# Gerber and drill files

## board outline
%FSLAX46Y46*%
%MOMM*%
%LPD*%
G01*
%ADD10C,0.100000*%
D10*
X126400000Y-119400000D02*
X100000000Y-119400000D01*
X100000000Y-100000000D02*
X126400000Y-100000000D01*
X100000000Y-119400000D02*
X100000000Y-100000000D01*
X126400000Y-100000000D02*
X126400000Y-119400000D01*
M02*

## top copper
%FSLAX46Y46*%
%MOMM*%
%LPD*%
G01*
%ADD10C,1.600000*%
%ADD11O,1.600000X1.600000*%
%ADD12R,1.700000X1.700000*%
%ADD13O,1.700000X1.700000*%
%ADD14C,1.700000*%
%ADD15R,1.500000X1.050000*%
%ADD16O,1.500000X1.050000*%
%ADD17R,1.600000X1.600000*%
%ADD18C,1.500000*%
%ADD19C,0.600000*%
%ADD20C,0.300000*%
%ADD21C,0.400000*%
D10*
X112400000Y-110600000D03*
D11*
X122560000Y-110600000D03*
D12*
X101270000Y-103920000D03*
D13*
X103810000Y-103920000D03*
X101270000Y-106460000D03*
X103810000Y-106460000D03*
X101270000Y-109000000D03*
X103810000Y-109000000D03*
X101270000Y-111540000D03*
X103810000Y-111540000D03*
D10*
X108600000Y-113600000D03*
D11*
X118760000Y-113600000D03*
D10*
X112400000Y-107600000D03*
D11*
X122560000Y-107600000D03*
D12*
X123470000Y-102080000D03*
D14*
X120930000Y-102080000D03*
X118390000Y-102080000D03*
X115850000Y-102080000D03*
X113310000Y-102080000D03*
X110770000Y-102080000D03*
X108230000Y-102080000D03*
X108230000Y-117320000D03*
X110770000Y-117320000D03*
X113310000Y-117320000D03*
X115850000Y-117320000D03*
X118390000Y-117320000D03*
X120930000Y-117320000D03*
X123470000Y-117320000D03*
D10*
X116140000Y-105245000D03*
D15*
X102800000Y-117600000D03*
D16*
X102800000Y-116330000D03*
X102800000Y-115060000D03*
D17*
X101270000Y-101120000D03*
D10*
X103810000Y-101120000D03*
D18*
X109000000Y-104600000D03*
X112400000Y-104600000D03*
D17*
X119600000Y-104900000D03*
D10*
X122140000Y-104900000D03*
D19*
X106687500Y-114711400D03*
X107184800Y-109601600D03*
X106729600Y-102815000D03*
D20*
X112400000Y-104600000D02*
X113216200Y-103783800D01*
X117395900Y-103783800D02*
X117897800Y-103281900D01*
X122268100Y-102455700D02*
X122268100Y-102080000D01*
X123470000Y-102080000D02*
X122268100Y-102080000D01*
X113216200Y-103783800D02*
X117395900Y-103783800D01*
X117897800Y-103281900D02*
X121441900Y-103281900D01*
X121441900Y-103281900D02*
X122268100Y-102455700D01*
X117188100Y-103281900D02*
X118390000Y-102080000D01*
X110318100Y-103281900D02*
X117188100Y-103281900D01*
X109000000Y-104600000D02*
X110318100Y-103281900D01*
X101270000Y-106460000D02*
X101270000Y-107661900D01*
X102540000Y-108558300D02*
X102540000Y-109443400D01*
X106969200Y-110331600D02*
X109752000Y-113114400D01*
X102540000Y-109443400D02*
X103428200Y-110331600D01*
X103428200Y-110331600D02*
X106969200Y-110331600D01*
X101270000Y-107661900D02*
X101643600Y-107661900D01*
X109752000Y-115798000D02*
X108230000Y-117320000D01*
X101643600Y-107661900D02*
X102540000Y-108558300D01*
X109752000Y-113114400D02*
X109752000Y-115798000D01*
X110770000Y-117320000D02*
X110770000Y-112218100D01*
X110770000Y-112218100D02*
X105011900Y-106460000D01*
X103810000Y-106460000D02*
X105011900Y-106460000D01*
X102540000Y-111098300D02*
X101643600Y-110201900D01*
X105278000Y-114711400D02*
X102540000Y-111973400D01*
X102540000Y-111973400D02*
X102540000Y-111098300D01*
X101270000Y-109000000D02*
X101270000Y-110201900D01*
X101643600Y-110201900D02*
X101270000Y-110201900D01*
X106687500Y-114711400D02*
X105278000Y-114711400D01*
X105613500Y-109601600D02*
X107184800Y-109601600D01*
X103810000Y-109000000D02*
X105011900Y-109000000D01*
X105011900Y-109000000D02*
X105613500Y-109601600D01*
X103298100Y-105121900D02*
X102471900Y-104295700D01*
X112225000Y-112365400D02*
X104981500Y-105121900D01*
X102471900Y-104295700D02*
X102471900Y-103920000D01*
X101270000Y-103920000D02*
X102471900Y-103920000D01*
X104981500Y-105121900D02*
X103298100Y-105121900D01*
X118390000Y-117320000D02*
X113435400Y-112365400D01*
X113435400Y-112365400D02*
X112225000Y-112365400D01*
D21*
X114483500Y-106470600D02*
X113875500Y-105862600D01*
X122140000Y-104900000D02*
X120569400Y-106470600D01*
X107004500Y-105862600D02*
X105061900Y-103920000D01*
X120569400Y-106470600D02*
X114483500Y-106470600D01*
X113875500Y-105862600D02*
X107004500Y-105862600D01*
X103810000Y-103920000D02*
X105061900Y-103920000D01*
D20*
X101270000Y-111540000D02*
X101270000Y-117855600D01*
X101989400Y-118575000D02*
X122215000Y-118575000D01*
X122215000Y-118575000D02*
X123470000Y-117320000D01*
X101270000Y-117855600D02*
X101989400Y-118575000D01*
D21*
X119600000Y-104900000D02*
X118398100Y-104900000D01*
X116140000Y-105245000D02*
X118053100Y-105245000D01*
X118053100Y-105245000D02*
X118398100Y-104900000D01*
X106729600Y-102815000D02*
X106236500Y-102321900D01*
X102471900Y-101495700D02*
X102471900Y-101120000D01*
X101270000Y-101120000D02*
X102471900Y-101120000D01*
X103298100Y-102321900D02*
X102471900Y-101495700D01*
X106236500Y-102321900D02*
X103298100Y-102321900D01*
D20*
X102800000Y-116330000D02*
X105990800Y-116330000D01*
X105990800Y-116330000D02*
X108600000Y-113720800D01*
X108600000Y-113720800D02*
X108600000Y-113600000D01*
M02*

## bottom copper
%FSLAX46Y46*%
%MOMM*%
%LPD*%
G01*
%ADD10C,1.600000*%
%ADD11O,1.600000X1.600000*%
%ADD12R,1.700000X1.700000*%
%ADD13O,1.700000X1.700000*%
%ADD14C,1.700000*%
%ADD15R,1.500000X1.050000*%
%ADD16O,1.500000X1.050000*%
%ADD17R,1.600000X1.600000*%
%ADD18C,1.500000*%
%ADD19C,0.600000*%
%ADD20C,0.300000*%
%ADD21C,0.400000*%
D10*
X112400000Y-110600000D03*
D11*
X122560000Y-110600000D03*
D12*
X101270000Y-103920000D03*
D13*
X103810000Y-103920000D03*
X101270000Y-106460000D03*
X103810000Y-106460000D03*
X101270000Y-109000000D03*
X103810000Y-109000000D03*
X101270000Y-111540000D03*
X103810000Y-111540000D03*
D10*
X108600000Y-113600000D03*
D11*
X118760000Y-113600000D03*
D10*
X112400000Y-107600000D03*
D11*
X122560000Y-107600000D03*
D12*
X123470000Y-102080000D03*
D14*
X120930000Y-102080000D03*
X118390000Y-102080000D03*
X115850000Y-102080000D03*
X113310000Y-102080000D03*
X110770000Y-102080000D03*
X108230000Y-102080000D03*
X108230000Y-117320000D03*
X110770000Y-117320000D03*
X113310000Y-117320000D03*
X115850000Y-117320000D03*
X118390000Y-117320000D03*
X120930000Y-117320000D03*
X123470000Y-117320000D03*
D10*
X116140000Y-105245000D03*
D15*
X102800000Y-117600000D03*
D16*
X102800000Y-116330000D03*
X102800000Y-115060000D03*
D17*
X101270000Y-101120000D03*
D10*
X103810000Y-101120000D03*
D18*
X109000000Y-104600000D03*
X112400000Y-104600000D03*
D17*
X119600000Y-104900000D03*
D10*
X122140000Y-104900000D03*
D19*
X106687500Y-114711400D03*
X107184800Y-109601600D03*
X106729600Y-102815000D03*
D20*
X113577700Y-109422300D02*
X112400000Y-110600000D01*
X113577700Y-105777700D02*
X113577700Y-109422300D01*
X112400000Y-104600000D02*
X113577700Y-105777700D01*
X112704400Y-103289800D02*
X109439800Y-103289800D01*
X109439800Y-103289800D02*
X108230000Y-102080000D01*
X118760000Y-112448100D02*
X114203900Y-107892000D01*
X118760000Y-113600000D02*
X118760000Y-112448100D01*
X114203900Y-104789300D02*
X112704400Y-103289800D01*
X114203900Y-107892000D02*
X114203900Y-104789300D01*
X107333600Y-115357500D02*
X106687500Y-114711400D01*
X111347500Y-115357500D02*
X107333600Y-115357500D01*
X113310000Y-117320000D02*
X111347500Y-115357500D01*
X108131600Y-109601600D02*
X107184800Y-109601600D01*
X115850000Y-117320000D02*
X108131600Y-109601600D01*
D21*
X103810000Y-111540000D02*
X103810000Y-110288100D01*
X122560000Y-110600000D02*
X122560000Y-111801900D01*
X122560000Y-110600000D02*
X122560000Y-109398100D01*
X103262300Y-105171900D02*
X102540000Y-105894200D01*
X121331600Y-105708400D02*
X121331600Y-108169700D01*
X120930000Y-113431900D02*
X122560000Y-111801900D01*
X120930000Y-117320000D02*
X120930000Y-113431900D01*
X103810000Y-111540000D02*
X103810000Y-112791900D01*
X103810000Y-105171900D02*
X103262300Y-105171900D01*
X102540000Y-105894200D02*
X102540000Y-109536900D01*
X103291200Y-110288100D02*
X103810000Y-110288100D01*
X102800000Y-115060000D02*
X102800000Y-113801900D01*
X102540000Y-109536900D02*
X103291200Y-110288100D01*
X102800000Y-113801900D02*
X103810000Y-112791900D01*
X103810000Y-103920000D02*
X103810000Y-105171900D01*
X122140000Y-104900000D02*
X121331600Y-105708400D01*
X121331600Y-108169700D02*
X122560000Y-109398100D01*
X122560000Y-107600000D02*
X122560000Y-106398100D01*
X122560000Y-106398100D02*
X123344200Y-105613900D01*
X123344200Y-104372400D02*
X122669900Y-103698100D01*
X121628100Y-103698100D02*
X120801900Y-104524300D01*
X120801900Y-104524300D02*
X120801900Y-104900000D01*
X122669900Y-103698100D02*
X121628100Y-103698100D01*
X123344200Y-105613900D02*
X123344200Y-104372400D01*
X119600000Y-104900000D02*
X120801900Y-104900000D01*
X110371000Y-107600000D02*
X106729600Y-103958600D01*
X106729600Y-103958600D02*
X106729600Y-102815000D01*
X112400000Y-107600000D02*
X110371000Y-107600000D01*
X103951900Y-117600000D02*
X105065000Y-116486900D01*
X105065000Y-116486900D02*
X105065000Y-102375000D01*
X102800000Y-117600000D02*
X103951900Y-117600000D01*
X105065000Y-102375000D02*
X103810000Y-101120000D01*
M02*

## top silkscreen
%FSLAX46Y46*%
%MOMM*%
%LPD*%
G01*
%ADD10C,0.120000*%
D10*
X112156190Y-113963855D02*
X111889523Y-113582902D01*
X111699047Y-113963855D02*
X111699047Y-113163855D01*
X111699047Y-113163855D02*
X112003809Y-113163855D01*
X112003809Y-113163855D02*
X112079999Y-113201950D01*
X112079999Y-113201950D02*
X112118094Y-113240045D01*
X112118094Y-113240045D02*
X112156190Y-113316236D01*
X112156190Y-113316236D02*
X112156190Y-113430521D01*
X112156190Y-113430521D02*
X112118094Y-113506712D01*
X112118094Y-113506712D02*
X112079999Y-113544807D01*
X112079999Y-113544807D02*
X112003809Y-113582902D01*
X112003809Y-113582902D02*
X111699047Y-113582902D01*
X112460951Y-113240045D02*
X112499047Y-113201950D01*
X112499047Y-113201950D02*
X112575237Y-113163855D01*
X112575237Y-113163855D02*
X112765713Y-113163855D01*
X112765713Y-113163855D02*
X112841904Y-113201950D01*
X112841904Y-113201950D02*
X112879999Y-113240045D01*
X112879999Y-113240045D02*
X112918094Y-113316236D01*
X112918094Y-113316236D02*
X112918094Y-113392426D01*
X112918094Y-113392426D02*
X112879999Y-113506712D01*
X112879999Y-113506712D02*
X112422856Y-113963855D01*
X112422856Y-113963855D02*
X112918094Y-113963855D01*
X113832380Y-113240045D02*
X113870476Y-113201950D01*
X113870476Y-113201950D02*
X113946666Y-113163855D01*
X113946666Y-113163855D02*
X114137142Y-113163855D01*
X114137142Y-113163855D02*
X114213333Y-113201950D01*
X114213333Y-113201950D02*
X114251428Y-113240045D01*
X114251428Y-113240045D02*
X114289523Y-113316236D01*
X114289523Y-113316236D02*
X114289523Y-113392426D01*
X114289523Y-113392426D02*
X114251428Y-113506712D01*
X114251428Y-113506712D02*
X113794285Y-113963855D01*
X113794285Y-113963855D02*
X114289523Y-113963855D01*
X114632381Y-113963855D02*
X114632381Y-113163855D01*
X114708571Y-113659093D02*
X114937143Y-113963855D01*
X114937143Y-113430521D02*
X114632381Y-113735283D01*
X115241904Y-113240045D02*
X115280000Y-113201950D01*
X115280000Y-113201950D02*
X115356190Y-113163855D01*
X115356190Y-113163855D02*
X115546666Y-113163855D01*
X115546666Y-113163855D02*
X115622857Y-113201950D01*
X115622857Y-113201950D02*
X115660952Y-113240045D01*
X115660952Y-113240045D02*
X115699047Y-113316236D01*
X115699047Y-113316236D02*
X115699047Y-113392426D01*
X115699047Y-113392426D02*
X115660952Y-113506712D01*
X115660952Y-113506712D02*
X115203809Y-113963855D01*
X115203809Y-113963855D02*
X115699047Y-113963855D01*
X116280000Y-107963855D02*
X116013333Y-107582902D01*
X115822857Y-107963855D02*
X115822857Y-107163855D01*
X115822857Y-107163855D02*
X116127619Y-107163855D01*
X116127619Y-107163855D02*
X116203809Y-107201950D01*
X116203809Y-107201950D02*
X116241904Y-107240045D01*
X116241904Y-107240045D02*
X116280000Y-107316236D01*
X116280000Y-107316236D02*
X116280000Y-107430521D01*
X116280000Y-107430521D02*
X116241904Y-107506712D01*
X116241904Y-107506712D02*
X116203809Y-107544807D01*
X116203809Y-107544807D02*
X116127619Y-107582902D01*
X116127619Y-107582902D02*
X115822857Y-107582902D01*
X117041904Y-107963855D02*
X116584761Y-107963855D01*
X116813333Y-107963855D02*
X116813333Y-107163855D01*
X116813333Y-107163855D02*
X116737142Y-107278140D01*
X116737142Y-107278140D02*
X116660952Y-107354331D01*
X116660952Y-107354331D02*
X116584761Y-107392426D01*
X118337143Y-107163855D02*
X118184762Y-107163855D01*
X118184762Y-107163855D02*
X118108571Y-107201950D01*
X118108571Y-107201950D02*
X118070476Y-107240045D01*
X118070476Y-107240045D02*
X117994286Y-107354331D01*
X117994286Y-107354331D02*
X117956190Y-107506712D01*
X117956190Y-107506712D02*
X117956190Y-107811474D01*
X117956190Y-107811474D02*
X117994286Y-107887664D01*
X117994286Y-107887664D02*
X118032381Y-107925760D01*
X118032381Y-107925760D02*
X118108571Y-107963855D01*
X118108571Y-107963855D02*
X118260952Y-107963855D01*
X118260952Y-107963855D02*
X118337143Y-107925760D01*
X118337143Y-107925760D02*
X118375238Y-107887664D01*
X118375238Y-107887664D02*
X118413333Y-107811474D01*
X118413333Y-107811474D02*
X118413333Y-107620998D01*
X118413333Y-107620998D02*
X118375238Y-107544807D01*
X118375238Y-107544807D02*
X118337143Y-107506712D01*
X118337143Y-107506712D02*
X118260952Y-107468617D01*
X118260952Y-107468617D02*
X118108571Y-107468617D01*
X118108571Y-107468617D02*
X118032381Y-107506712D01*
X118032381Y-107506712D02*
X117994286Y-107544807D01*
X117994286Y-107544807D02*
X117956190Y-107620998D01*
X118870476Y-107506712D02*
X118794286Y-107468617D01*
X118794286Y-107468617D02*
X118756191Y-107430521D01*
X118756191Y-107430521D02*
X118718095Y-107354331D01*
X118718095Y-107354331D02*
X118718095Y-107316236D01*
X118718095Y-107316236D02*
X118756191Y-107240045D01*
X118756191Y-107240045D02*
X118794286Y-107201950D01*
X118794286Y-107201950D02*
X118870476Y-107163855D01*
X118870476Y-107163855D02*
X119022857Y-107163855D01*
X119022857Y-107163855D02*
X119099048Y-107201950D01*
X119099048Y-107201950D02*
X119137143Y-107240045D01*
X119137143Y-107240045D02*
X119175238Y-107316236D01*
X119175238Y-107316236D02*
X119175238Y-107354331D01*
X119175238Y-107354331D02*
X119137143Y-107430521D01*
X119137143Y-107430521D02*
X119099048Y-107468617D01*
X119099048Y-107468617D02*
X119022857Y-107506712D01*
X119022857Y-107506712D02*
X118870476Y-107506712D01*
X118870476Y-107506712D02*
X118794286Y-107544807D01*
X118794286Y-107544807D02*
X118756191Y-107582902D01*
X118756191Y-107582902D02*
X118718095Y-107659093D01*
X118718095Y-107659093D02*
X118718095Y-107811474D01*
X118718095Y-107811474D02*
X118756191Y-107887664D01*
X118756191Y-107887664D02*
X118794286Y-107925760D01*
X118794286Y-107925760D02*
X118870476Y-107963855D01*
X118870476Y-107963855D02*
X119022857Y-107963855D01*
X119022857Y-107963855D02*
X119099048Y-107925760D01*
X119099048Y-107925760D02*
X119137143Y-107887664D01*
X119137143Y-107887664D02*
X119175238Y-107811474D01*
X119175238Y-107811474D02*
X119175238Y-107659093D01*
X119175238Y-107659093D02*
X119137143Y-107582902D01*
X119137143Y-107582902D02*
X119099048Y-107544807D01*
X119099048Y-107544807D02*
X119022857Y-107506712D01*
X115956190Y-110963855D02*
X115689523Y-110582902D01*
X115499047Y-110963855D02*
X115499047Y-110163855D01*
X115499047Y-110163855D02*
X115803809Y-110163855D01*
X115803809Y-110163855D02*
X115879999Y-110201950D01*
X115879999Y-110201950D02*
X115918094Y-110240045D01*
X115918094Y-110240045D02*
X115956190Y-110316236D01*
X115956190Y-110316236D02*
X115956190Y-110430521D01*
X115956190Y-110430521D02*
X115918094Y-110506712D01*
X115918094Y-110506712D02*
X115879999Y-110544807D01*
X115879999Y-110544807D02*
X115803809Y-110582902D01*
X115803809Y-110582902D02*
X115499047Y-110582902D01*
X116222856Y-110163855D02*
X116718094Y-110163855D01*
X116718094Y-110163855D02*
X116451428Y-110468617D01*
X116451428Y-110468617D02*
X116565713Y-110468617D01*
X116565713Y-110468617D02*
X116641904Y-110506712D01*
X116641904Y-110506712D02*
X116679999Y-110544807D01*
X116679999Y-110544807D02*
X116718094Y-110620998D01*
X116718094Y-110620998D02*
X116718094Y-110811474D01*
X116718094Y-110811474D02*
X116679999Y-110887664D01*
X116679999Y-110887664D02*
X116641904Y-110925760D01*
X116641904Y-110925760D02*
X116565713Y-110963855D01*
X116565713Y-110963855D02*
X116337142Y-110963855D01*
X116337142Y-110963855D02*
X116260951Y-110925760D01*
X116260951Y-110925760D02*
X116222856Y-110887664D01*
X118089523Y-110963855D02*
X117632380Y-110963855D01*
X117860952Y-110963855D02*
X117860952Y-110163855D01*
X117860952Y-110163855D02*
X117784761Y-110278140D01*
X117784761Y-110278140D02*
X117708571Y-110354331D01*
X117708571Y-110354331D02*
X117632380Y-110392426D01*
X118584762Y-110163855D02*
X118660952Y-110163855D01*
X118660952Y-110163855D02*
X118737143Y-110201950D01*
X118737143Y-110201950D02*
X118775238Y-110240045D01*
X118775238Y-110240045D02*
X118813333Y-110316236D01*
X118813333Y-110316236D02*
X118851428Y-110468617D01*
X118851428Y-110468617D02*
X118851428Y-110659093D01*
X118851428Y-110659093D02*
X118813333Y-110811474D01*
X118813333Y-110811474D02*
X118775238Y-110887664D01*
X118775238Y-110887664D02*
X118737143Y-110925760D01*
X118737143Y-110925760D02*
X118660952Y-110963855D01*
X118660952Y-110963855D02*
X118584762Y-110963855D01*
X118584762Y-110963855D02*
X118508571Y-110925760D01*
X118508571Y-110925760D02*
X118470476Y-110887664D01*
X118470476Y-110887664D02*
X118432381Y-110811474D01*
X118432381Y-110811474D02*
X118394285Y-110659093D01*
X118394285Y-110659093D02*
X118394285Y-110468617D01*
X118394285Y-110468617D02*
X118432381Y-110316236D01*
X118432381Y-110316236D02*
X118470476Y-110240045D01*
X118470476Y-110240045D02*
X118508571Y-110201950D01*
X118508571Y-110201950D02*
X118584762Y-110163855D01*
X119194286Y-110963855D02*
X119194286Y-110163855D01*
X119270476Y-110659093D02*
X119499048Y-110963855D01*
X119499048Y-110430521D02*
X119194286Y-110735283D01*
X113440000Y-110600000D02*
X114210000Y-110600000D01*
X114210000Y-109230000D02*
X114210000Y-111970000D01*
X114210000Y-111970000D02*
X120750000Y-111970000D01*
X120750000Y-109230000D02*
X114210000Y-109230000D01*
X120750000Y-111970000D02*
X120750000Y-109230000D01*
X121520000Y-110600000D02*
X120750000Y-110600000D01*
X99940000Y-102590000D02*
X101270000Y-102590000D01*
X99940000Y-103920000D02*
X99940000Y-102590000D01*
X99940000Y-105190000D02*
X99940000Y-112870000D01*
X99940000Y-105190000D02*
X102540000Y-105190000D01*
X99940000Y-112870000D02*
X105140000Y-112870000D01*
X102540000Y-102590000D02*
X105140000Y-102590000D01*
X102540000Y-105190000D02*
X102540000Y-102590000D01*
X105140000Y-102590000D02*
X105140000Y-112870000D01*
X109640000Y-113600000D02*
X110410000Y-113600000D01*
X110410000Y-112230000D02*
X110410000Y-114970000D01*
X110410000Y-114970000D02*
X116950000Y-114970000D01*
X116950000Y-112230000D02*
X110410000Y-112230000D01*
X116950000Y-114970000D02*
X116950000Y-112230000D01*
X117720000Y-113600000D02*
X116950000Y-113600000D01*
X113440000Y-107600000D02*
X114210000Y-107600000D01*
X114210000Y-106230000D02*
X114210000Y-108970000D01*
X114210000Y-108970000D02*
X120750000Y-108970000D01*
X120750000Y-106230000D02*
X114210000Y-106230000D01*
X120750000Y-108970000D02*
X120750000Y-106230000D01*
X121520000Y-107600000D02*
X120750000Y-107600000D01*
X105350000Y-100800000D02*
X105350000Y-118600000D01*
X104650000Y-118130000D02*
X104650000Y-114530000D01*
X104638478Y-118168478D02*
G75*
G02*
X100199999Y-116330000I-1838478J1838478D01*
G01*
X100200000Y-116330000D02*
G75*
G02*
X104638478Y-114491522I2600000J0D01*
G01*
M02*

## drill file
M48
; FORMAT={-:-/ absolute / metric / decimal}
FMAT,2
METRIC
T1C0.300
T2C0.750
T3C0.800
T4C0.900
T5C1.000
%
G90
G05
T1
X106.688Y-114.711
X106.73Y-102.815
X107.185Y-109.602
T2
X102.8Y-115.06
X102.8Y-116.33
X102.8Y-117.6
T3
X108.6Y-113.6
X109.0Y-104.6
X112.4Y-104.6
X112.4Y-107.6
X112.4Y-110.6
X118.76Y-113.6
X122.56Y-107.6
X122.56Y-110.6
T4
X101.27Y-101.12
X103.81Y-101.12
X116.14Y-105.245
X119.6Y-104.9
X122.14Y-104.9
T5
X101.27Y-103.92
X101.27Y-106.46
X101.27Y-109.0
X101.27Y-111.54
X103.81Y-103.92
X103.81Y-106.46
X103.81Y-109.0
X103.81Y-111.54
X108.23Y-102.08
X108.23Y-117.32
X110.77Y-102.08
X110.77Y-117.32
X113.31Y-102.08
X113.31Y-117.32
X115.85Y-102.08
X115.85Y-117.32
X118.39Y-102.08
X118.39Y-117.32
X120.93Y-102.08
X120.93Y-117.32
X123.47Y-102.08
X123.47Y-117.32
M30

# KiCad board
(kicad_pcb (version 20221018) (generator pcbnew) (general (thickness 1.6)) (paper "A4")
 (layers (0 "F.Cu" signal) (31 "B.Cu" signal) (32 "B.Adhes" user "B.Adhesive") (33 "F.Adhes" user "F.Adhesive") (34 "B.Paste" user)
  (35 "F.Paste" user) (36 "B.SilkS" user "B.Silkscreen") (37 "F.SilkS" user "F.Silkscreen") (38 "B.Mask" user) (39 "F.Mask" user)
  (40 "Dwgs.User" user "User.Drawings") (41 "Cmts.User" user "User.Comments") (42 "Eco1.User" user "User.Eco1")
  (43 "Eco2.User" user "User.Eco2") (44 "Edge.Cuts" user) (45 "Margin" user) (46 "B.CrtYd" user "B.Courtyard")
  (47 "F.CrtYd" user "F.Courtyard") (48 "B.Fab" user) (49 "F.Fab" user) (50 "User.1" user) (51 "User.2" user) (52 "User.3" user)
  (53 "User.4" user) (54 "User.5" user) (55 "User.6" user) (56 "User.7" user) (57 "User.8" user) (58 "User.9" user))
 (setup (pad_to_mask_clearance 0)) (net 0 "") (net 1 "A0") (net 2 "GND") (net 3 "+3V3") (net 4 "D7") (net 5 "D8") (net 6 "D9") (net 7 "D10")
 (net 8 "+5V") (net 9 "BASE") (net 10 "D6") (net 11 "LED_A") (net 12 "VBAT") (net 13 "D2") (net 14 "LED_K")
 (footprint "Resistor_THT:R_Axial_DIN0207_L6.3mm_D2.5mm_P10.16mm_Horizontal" (layer "F.Cu") (at 112.4 110.6)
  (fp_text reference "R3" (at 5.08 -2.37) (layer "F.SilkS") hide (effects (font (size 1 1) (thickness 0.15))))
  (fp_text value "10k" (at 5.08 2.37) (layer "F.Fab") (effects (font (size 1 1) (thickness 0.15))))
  (fp_line (start 1.04 0) (end 1.81 0) (stroke (width 0.12) (type solid)) (layer "F.SilkS"))
  (fp_line (start 1.81 -1.37) (end 1.81 1.37) (stroke (width 0.12) (type solid)) (layer "F.SilkS"))
  (fp_line (start 1.81 1.37) (end 8.35 1.37) (stroke (width 0.12) (type solid)) (layer "F.SilkS"))
  (fp_line (start 8.35 -1.37) (end 1.81 -1.37) (stroke (width 0.12) (type solid)) (layer "F.SilkS"))
  (fp_line (start 8.35 1.37) (end 8.35 -1.37) (stroke (width 0.12) (type solid)) (layer "F.SilkS"))
  (fp_line (start 9.12 0) (end 8.35 0) (stroke (width 0.12) (type solid)) (layer "F.SilkS"))
  (pad "1" thru_hole circle (at 0 0) (size 1.6 1.6) (drill 0.8) (layers "*.Cu" "*.Mask") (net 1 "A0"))
  (pad "2" thru_hole oval (at 10.16 0) (size 1.6 1.6) (drill 0.8) (layers "*.Cu" "*.Mask") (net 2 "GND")))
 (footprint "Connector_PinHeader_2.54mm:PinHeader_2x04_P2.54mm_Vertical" (layer "F.Cu") (at 101.27 103.92)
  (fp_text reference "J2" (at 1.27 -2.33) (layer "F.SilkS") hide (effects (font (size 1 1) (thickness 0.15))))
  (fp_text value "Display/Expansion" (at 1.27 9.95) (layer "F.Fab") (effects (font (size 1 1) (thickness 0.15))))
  (fp_line (start -1.33 -1.33) (end 0 -1.33) (stroke (width 0.12) (type solid)) (layer "F.SilkS"))
  (fp_line (start -1.33 0) (end -1.33 -1.33) (stroke (width 0.12) (type solid)) (layer "F.SilkS"))
  (fp_line (start -1.33 1.27) (end -1.33 8.95) (stroke (width 0.12) (type solid)) (layer "F.SilkS"))
  (fp_line (start -1.33 1.27) (end 1.27 1.27) (stroke (width 0.12) (type solid)) (layer "F.SilkS"))
  (fp_line (start -1.33 8.95) (end 3.87 8.95) (stroke (width 0.12) (type solid)) (layer "F.SilkS"))
  (fp_line (start 1.27 -1.33) (end 3.87 -1.33) (stroke (width 0.12) (type solid)) (layer "F.SilkS"))
  (fp_line (start 1.27 1.27) (end 1.27 -1.33) (stroke (width 0.12) (type solid)) (layer "F.SilkS"))
  (fp_line (start 3.87 -1.33) (end 3.87 8.95) (stroke (width 0.12) (type solid)) (layer "F.SilkS"))
  (pad "1" thru_hole rect (at 0 0) (size 1.7 1.7) (drill 1) (layers "*.Cu" "*.Mask") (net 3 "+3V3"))
  (pad "2" thru_hole oval (at 2.54 0) (size 1.7 1.7) (drill 1) (layers "*.Cu" "*.Mask") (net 2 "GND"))
  (pad "3" thru_hole oval (at 0 2.54) (size 1.7 1.7) (drill 1) (layers "*.Cu" "*.Mask") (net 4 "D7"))
  (pad "4" thru_hole oval (at 2.54 2.54) (size 1.7 1.7) (drill 1) (layers "*.Cu" "*.Mask") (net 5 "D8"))
  (pad "5" thru_hole oval (at 0 5.08) (size 1.7 1.7) (drill 1) (layers "*.Cu" "*.Mask") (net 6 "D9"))
  (pad "6" thru_hole oval (at 2.54 5.08) (size 1.7 1.7) (drill 1) (layers "*.Cu" "*.Mask") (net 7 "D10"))
  (pad "7" thru_hole oval (at 0 7.62) (size 1.7 1.7) (drill 1) (layers "*.Cu" "*.Mask") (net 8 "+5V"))
  (pad "8" thru_hole oval (at 2.54 7.62) (size 1.7 1.7) (drill 1) (layers "*.Cu" "*.Mask") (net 2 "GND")))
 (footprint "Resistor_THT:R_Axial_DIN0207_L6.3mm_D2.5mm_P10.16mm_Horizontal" (layer "F.Cu") (at 108.6 113.6)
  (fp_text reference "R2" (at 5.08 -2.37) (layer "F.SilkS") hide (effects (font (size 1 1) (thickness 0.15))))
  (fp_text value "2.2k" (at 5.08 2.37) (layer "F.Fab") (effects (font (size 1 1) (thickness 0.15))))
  (fp_line (start 1.04 0) (end 1.81 0) (stroke (width 0.12) (type solid)) (layer "F.SilkS"))
  (fp_line (start 1.81 -1.37) (end 1.81 1.37) (stroke (width 0.12) (type solid)) (layer "F.SilkS"))
  (fp_line (start 1.81 1.37) (end 8.35 1.37) (stroke (width 0.12) (type solid)) (layer "F.SilkS"))
  (fp_line (start 8.35 -1.37) (end 1.81 -1.37) (stroke (width 0.12) (type solid)) (layer "F.SilkS"))
  (fp_line (start 8.35 1.37) (end 8.35 -1.37) (stroke (width 0.12) (type solid)) (layer "F.SilkS"))
  (fp_line (start 9.12 0) (end 8.35 0) (stroke (width 0.12) (type solid)) (layer "F.SilkS"))
  (pad "1" thru_hole circle (at 0 0) (size 1.6 1.6) (drill 0.8) (layers "*.Cu" "*.Mask") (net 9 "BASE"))
  (pad "2" thru_hole oval (at 10.16 0) (size 1.6 1.6) (drill 0.8) (layers "*.Cu" "*.Mask") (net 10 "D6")))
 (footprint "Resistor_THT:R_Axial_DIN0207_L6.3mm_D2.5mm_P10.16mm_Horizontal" (layer "F.Cu") (at 112.4 107.6)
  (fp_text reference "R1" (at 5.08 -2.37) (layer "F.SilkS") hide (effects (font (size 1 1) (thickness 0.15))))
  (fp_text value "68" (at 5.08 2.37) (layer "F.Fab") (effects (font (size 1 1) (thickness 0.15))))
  (fp_line (start 1.04 0) (end 1.81 0) (stroke (width 0.12) (type solid)) (layer "F.SilkS"))
  (fp_line (start 1.81 -1.37) (end 1.81 1.37) (stroke (width 0.12) (type solid)) (layer "F.SilkS"))
  (fp_line (start 1.81 1.37) (end 8.35 1.37) (stroke (width 0.12) (type solid)) (layer "F.SilkS"))
  (fp_line (start 8.35 -1.37) (end 1.81 -1.37) (stroke (width 0.12) (type solid)) (layer "F.SilkS"))
  (fp_line (start 8.35 1.37) (end 8.35 -1.37) (stroke (width 0.12) (type solid)) (layer "F.SilkS"))
  (fp_line (start 9.12 0) (end 8.35 0) (stroke (width 0.12) (type solid)) (layer "F.SilkS"))
  (pad "1" thru_hole circle (at 0 0) (size 1.6 1.6) (drill 0.8) (layers "*.Cu" "*.Mask") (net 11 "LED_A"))
  (pad "2" thru_hole oval (at 10.16 0) (size 1.6 1.6) (drill 0.8) (layers "*.Cu" "*.Mask") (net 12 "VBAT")))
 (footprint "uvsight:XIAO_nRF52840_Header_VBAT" (layer "F.Cu") (at 115.85 109.7)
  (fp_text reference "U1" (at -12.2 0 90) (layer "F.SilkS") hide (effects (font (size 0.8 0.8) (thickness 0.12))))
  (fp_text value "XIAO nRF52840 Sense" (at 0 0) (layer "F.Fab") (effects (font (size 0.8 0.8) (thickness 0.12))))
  (fp_line (start -10.5 -8.9) (end -10.5 8.9) (stroke (width 0.12) (type solid)) (layer "F.SilkS"))
  (pad "1" thru_hole rect (at 7.62 -7.62) (size 1.7 1.7) (drill 1) (layers "*.Cu" "*.Mask") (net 1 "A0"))
  (pad "2" thru_hole circle (at 5.08 -7.62) (size 1.7 1.7) (drill 1) (layers "*.Cu" "*.Mask"))
  (pad "3" thru_hole circle (at 2.54 -7.62) (size 1.7 1.7) (drill 1) (layers "*.Cu" "*.Mask") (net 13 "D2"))
  (pad "4" thru_hole circle (at 0 -7.62) (size 1.7 1.7) (drill 1) (layers "*.Cu" "*.Mask"))
  (pad "5" thru_hole circle (at -2.54 -7.62) (size 1.7 1.7) (drill 1) (layers "*.Cu" "*.Mask"))
  (pad "6" thru_hole circle (at -5.08 -7.62) (size 1.7 1.7) (drill 1) (layers "*.Cu" "*.Mask"))
  (pad "7" thru_hole circle (at -7.62 -7.62) (size 1.7 1.7) (drill 1) (layers "*.Cu" "*.Mask") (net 10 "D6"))
  (pad "8" thru_hole circle (at -7.62 7.62) (size 1.7 1.7) (drill 1) (layers "*.Cu" "*.Mask") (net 4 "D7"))
  (pad "9" thru_hole circle (at -5.08 7.62) (size 1.7 1.7) (drill 1) (layers "*.Cu" "*.Mask") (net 5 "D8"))
  (pad "10" thru_hole circle (at -2.54 7.62) (size 1.7 1.7) (drill 1) (layers "*.Cu" "*.Mask") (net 6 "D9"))
  (pad "11" thru_hole circle (at 0 7.62) (size 1.7 1.7) (drill 1) (layers "*.Cu" "*.Mask") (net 7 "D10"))
  (pad "12" thru_hole circle (at 2.54 7.62) (size 1.7 1.7) (drill 1) (layers "*.Cu" "*.Mask") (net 3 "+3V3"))
  (pad "13" thru_hole circle (at 5.08 7.62) (size 1.7 1.7) (drill 1) (layers "*.Cu" "*.Mask") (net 2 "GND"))
  (pad "14" thru_hole circle (at 7.62 7.62) (size 1.7 1.7) (drill 1) (layers "*.Cu" "*.Mask") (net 8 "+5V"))
  (pad "15" thru_hole circle (at 0.29 -4.455) (size 1.6 1.6) (drill 0.9) (layers "*.Cu" "*.Mask") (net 12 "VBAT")))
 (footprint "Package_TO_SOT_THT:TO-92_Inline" (layer "F.Cu") (at 102.8 117.6 90)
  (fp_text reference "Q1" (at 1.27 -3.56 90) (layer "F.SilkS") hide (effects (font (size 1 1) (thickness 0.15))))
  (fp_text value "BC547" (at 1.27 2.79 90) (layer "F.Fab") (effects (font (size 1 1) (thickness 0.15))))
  (fp_line (start -0.53 1.85) (end 3.07 1.85) (stroke (width 0.12) (type solid)) (layer "F.SilkS"))
  (fp_arc (start -0.568478 1.838478) (mid -1.132087 -0.994977) (end 1.27 -2.6) (stroke (width 0.12) (type solid)) (layer "F.SilkS"))
  (fp_arc (start 1.27 -2.6) (mid 3.672087 -0.994977) (end 3.108478 1.838478) (stroke (width 0.12) (type solid)) (layer "F.SilkS"))
  (pad "1" thru_hole rect (at 0 0 90) (size 1.05 1.5) (drill 0.75) (layers "*.Cu" "*.Mask") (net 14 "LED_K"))
  (pad "2" thru_hole oval (at 1.27 0 90) (size 1.05 1.5) (drill 0.75) (layers "*.Cu" "*.Mask") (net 9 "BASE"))
  (pad "3" thru_hole oval (at 2.54 0 90) (size 1.05 1.5) (drill 0.75) (layers "*.Cu" "*.Mask") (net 2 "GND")))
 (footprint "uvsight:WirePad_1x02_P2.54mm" (layer "F.Cu") (at 101.27 101.12)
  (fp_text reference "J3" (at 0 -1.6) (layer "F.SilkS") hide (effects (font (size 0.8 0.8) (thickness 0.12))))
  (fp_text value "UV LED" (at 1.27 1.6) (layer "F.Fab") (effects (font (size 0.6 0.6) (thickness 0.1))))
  (pad "1" thru_hole rect (at 0 0) (size 1.6 1.6) (drill 0.9) (layers "*.Cu" "*.Mask") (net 11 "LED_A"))
  (pad "2" thru_hole circle (at 2.54 0) (size 1.6 1.6) (drill 0.9) (layers "*.Cu" "*.Mask") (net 14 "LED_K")))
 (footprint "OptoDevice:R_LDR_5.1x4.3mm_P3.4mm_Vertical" (layer "B.Cu") (at 109 104.6)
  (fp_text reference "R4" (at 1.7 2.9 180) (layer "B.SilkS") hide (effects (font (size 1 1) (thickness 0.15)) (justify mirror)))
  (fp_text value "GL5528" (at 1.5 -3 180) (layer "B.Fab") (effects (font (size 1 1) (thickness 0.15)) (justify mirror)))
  (pad "1" thru_hole circle (at 0 0) (size 1.5 1.5) (drill 0.8) (layers "*.Cu" "*.Mask") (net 13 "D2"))
  (pad "2" thru_hole circle (at 3.4 0) (size 1.5 1.5) (drill 0.8) (layers "*.Cu" "*.Mask") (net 1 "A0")))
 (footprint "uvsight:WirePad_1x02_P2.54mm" (layer "B.Cu") (at 119.6 104.9)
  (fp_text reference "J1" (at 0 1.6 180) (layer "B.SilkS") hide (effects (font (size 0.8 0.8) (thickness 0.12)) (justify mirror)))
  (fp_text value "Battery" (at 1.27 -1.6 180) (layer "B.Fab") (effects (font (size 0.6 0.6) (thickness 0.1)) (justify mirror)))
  (pad "1" thru_hole rect (at 0 0) (size 1.6 1.6) (drill 0.9) (layers "*.Cu" "*.Mask") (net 12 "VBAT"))
  (pad "2" thru_hole circle (at 2.54 0) (size 1.6 1.6) (drill 0.9) (layers "*.Cu" "*.Mask") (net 2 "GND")))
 (gr_line (start 126.4 119.4) (end 100 119.4) (stroke (width 0.1) (type default)) (layer "Edge.Cuts"))
 (gr_line (start 100 100) (end 126.4 100) (stroke (width 0.1) (type default)) (layer "Edge.Cuts"))
 (gr_line (start 100 119.4) (end 100 100) (stroke (width 0.1) (type default)) (layer "Edge.Cuts"))
 (gr_line (start 126.4 100) (end 126.4 119.4) (stroke (width 0.1) (type default)) (layer "Edge.Cuts"))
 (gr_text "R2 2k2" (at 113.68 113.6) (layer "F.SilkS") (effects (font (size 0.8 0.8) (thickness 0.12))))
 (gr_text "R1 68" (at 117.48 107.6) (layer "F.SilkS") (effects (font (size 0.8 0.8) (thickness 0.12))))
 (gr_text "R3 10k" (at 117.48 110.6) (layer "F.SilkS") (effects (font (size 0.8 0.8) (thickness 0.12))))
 (segment (start 112.4 104.6) (end 113.2162 103.7838) (width 0.3) (layer "F.Cu") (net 1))
 (segment (start 117.3959 103.7838) (end 117.8978 103.2819) (width 0.3) (layer "F.Cu") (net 1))
 (segment (start 122.2681 102.4557) (end 122.2681 102.08) (width 0.3) (layer "F.Cu") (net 1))
 (segment (start 123.47 102.08) (end 122.2681 102.08) (width 0.3) (layer "F.Cu") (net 1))
 (segment (start 113.2162 103.7838) (end 117.3959 103.7838) (width 0.3) (layer "F.Cu") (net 1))
 (segment (start 117.8978 103.2819) (end 121.4419 103.2819) (width 0.3) (layer "F.Cu") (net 1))
 (segment (start 121.4419 103.2819) (end 122.2681 102.4557) (width 0.3) (layer "F.Cu") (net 1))
 (segment (start 113.5777 109.4223) (end 112.4 110.6) (width 0.3) (layer "B.Cu") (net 1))
 (segment (start 113.5777 105.7777) (end 113.5777 109.4223) (width 0.3) (layer "B.Cu") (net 1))
 (segment (start 112.4 104.6) (end 113.5777 105.7777) (width 0.3) (layer "B.Cu") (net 1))
 (segment (start 117.1881 103.2819) (end 118.39 102.08) (width 0.3) (layer "F.Cu") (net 13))
 (segment (start 110.3181 103.2819) (end 117.1881 103.2819) (width 0.3) (layer "F.Cu") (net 13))
 (segment (start 109 104.6) (end 110.3181 103.2819) (width 0.3) (layer "F.Cu") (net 13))
 (segment (start 112.7044 103.2898) (end 109.4398 103.2898) (width 0.3) (layer "B.Cu") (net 10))
 (segment (start 109.4398 103.2898) (end 108.23 102.08) (width 0.3) (layer "B.Cu") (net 10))
 (segment (start 118.76 112.4481) (end 114.2039 107.892) (width 0.3) (layer "B.Cu") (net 10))
 (segment (start 118.76 113.6) (end 118.76 112.4481) (width 0.3) (layer "B.Cu") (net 10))
 (segment (start 114.2039 104.7893) (end 112.7044 103.2898) (width 0.3) (layer "B.Cu") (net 10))
 (segment (start 114.2039 107.892) (end 114.2039 104.7893) (width 0.3) (layer "B.Cu") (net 10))
 (segment (start 101.27 106.46) (end 101.27 107.6619) (width 0.3) (layer "F.Cu") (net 4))
 (segment (start 102.54 108.5583) (end 102.54 109.4434) (width 0.3) (layer "F.Cu") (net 4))
 (segment (start 106.9692 110.3316) (end 109.752 113.1144) (width 0.3) (layer "F.Cu") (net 4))
 (segment (start 102.54 109.4434) (end 103.4282 110.3316) (width 0.3) (layer "F.Cu") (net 4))
 (segment (start 103.4282 110.3316) (end 106.9692 110.3316) (width 0.3) (layer "F.Cu") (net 4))
 (segment (start 101.27 107.6619) (end 101.6436 107.6619) (width 0.3) (layer "F.Cu") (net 4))
 (segment (start 109.752 115.798) (end 108.23 117.32) (width 0.3) (layer "F.Cu") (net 4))
 (segment (start 101.6436 107.6619) (end 102.54 108.5583) (width 0.3) (layer "F.Cu") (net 4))
 (segment (start 109.752 113.1144) (end 109.752 115.798) (width 0.3) (layer "F.Cu") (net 4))
 (segment (start 110.77 117.32) (end 110.77 112.2181) (width 0.3) (layer "F.Cu") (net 5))
 (segment (start 110.77 112.2181) (end 105.0119 106.46) (width 0.3) (layer "F.Cu") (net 5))
 (segment (start 103.81 106.46) (end 105.0119 106.46) (width 0.3) (layer "F.Cu") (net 5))
 (segment (start 102.54 111.0983) (end 101.6436 110.2019) (width 0.3) (layer "F.Cu") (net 6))
 (segment (start 105.278 114.7114) (end 102.54 111.9734) (width 0.3) (layer "F.Cu") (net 6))
 (segment (start 102.54 111.9734) (end 102.54 111.0983) (width 0.3) (layer "F.Cu") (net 6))
 (segment (start 101.27 109) (end 101.27 110.2019) (width 0.3) (layer "F.Cu") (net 6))
 (segment (start 101.6436 110.2019) (end 101.27 110.2019) (width 0.3) (layer "F.Cu") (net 6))
 (segment (start 106.6875 114.7114) (end 105.278 114.7114) (width 0.3) (layer "F.Cu") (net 6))
 (via (at 106.6875 114.7114) (size 0.6) (drill 0.3) (layers "F.Cu" "B.Cu") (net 6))
 (segment (start 107.3336 115.3575) (end 106.6875 114.7114) (width 0.3) (layer "B.Cu") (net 6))
 (segment (start 111.3475 115.3575) (end 107.3336 115.3575) (width 0.3) (layer "B.Cu") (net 6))
 (segment (start 113.31 117.32) (end 111.3475 115.3575) (width 0.3) (layer "B.Cu") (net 6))
 (segment (start 105.6135 109.6016) (end 107.1848 109.6016) (width 0.3) (layer "F.Cu") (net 7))
 (segment (start 103.81 109) (end 105.0119 109) (width 0.3) (layer "F.Cu") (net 7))
 (segment (start 105.0119 109) (end 105.6135 109.6016) (width 0.3) (layer "F.Cu") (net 7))
 (via (at 107.1848 109.6016) (size 0.6) (drill 0.3) (layers "F.Cu" "B.Cu") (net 7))
 (segment (start 108.1316 109.6016) (end 107.1848 109.6016) (width 0.3) (layer "B.Cu") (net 7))
 (segment (start 115.85 117.32) (end 108.1316 109.6016) (width 0.3) (layer "B.Cu") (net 7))
 (segment (start 103.2981 105.1219) (end 102.4719 104.2957) (width 0.3) (layer "F.Cu") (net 3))
 (segment (start 112.225 112.3654) (end 104.9815 105.1219) (width 0.3) (layer "F.Cu") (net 3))
 (segment (start 102.4719 104.2957) (end 102.4719 103.92) (width 0.3) (layer "F.Cu") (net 3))
 (segment (start 101.27 103.92) (end 102.4719 103.92) (width 0.3) (layer "F.Cu") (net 3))
 (segment (start 104.9815 105.1219) (end 103.2981 105.1219) (width 0.3) (layer "F.Cu") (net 3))
 (segment (start 118.39 117.32) (end 113.4354 112.3654) (width 0.3) (layer "F.Cu") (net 3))
 (segment (start 113.4354 112.3654) (end 112.225 112.3654) (width 0.3) (layer "F.Cu") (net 3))
 (segment (start 114.4835 106.4706) (end 113.8755 105.8626) (width 0.4) (layer "F.Cu") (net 2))
 (segment (start 122.14 104.9) (end 120.5694 106.4706) (width 0.4) (layer "F.Cu") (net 2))
 (segment (start 107.0045 105.8626) (end 105.0619 103.92) (width 0.4) (layer "F.Cu") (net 2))
 (segment (start 120.5694 106.4706) (end 114.4835 106.4706) (width 0.4) (layer "F.Cu") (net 2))
 (segment (start 113.8755 105.8626) (end 107.0045 105.8626) (width 0.4) (layer "F.Cu") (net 2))
 (segment (start 103.81 103.92) (end 105.0619 103.92) (width 0.4) (layer "F.Cu") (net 2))
 (segment (start 103.81 111.54) (end 103.81 110.2881) (width 0.4) (layer "B.Cu") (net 2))
 (segment (start 122.56 110.6) (end 122.56 111.8019) (width 0.4) (layer "B.Cu") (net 2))
 (segment (start 122.56 110.6) (end 122.56 109.3981) (width 0.4) (layer "B.Cu") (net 2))
 (segment (start 103.2623 105.1719) (end 102.54 105.8942) (width 0.4) (layer "B.Cu") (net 2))
 (segment (start 121.3316 105.7084) (end 121.3316 108.1697) (width 0.4) (layer "B.Cu") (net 2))
 (segment (start 120.93 113.4319) (end 122.56 111.8019) (width 0.4) (layer "B.Cu") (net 2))
 (segment (start 120.93 117.32) (end 120.93 113.4319) (width 0.4) (layer "B.Cu") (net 2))
 (segment (start 103.81 111.54) (end 103.81 112.7919) (width 0.4) (layer "B.Cu") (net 2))
 (segment (start 103.81 105.1719) (end 103.2623 105.1719) (width 0.4) (layer "B.Cu") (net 2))
 (segment (start 102.54 105.8942) (end 102.54 109.5369) (width 0.4) (layer "B.Cu") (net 2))
 (segment (start 103.2912 110.2881) (end 103.81 110.2881) (width 0.4) (layer "B.Cu") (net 2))
 (segment (start 102.8 115.06) (end 102.8 113.8019) (width 0.4) (layer "B.Cu") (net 2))
 (segment (start 102.54 109.5369) (end 103.2912 110.2881) (width 0.4) (layer "B.Cu") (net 2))
 (segment (start 102.8 113.8019) (end 103.81 112.7919) (width 0.4) (layer "B.Cu") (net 2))
 (segment (start 103.81 103.92) (end 103.81 105.1719) (width 0.4) (layer "B.Cu") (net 2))
 (segment (start 122.14 104.9) (end 121.3316 105.7084) (width 0.4) (layer "B.Cu") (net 2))
 (segment (start 121.3316 108.1697) (end 122.56 109.3981) (width 0.4) (layer "B.Cu") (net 2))
 (segment (start 101.27 111.54) (end 101.27 117.8556) (width 0.3) (layer "F.Cu") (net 8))
 (segment (start 101.9894 118.575) (end 122.215 118.575) (width 0.3) (layer "F.Cu") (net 8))
 (segment (start 122.215 118.575) (end 123.47 117.32) (width 0.3) (layer "F.Cu") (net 8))
 (segment (start 101.27 117.8556) (end 101.9894 118.575) (width 0.3) (layer "F.Cu") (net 8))
 (segment (start 119.6 104.9) (end 118.3981 104.9) (width 0.4) (layer "F.Cu") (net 12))
 (segment (start 116.14 105.245) (end 118.0531 105.245) (width 0.4) (layer "F.Cu") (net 12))
 (segment (start 118.0531 105.245) (end 118.3981 104.9) (width 0.4) (layer "F.Cu") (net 12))
 (segment (start 122.56 107.6) (end 122.56 106.3981) (width 0.4) (layer "B.Cu") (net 12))
 (segment (start 122.56 106.3981) (end 123.3442 105.6139) (width 0.4) (layer "B.Cu") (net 12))
 (segment (start 123.3442 104.3724) (end 122.6699 103.6981) (width 0.4) (layer "B.Cu") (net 12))
 (segment (start 121.6281 103.6981) (end 120.8019 104.5243) (width 0.4) (layer "B.Cu") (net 12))
 (segment (start 120.8019 104.5243) (end 120.8019 104.9) (width 0.4) (layer "B.Cu") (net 12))
 (segment (start 122.6699 103.6981) (end 121.6281 103.6981) (width 0.4) (layer "B.Cu") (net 12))
 (segment (start 123.3442 105.6139) (end 123.3442 104.3724) (width 0.4) (layer "B.Cu") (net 12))
 (segment (start 119.6 104.9) (end 120.8019 104.9) (width 0.4) (layer "B.Cu") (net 12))
 (segment (start 106.7296 102.815) (end 106.2365 102.3219) (width 0.4) (layer "F.Cu") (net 11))
 (segment (start 102.4719 101.4957) (end 102.4719 101.12) (width 0.4) (layer "F.Cu") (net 11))
 (segment (start 101.27 101.12) (end 102.4719 101.12) (width 0.4) (layer "F.Cu") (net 11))
 (segment (start 103.2981 102.3219) (end 102.4719 101.4957) (width 0.4) (layer "F.Cu") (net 11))
 (segment (start 106.2365 102.3219) (end 103.2981 102.3219) (width 0.4) (layer "F.Cu") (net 11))
 (via (at 106.7296 102.815) (size 0.6) (drill 0.3) (layers "F.Cu" "B.Cu") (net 11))
 (segment (start 110.371 107.6) (end 106.7296 103.9586) (width 0.4) (layer "B.Cu") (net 11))
 (segment (start 106.7296 103.9586) (end 106.7296 102.815) (width 0.4) (layer "B.Cu") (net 11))
 (segment (start 112.4 107.6) (end 110.371 107.6) (width 0.4) (layer "B.Cu") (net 11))
 (segment (start 102.8 116.33) (end 105.9908 116.33) (width 0.3) (layer "F.Cu") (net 9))
 (segment (start 105.9908 116.33) (end 108.6 113.7208) (width 0.3) (layer "F.Cu") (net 9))
 (segment (start 108.6 113.7208) (end 108.6 113.6) (width 0.3) (layer "F.Cu") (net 9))
 (segment (start 103.9519 117.6) (end 105.065 116.4869) (width 0.4) (layer "B.Cu") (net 14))
 (segment (start 105.065 116.4869) (end 105.065 102.375) (width 0.4) (layer "B.Cu") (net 14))
 (segment (start 102.8 117.6) (end 103.9519 117.6) (width 0.4) (layer "B.Cu") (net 14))
 (segment (start 105.065 102.375) (end 103.81 101.12) (width 0.4) (layer "B.Cu") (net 14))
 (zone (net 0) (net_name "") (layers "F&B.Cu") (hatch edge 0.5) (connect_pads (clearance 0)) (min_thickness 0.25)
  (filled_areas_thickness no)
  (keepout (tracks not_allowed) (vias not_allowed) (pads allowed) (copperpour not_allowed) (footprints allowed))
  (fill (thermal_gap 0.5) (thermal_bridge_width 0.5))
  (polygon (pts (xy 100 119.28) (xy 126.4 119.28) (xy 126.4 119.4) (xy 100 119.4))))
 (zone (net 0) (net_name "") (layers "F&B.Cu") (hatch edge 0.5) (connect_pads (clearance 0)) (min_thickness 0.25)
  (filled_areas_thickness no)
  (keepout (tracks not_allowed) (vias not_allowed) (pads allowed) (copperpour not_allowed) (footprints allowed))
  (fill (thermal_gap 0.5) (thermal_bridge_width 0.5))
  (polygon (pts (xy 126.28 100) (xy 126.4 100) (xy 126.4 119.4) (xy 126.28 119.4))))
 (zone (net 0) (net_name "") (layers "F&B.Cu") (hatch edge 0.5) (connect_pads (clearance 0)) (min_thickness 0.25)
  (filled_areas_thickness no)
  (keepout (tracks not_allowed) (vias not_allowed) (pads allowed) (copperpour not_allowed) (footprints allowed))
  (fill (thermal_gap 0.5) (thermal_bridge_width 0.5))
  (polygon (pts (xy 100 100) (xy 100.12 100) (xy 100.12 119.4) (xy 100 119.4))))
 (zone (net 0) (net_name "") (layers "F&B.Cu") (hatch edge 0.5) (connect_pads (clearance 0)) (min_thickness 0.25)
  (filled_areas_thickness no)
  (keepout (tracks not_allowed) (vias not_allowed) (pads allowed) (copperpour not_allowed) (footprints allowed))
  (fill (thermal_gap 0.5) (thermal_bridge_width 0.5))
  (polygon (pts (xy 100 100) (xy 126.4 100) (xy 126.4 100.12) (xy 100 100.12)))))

